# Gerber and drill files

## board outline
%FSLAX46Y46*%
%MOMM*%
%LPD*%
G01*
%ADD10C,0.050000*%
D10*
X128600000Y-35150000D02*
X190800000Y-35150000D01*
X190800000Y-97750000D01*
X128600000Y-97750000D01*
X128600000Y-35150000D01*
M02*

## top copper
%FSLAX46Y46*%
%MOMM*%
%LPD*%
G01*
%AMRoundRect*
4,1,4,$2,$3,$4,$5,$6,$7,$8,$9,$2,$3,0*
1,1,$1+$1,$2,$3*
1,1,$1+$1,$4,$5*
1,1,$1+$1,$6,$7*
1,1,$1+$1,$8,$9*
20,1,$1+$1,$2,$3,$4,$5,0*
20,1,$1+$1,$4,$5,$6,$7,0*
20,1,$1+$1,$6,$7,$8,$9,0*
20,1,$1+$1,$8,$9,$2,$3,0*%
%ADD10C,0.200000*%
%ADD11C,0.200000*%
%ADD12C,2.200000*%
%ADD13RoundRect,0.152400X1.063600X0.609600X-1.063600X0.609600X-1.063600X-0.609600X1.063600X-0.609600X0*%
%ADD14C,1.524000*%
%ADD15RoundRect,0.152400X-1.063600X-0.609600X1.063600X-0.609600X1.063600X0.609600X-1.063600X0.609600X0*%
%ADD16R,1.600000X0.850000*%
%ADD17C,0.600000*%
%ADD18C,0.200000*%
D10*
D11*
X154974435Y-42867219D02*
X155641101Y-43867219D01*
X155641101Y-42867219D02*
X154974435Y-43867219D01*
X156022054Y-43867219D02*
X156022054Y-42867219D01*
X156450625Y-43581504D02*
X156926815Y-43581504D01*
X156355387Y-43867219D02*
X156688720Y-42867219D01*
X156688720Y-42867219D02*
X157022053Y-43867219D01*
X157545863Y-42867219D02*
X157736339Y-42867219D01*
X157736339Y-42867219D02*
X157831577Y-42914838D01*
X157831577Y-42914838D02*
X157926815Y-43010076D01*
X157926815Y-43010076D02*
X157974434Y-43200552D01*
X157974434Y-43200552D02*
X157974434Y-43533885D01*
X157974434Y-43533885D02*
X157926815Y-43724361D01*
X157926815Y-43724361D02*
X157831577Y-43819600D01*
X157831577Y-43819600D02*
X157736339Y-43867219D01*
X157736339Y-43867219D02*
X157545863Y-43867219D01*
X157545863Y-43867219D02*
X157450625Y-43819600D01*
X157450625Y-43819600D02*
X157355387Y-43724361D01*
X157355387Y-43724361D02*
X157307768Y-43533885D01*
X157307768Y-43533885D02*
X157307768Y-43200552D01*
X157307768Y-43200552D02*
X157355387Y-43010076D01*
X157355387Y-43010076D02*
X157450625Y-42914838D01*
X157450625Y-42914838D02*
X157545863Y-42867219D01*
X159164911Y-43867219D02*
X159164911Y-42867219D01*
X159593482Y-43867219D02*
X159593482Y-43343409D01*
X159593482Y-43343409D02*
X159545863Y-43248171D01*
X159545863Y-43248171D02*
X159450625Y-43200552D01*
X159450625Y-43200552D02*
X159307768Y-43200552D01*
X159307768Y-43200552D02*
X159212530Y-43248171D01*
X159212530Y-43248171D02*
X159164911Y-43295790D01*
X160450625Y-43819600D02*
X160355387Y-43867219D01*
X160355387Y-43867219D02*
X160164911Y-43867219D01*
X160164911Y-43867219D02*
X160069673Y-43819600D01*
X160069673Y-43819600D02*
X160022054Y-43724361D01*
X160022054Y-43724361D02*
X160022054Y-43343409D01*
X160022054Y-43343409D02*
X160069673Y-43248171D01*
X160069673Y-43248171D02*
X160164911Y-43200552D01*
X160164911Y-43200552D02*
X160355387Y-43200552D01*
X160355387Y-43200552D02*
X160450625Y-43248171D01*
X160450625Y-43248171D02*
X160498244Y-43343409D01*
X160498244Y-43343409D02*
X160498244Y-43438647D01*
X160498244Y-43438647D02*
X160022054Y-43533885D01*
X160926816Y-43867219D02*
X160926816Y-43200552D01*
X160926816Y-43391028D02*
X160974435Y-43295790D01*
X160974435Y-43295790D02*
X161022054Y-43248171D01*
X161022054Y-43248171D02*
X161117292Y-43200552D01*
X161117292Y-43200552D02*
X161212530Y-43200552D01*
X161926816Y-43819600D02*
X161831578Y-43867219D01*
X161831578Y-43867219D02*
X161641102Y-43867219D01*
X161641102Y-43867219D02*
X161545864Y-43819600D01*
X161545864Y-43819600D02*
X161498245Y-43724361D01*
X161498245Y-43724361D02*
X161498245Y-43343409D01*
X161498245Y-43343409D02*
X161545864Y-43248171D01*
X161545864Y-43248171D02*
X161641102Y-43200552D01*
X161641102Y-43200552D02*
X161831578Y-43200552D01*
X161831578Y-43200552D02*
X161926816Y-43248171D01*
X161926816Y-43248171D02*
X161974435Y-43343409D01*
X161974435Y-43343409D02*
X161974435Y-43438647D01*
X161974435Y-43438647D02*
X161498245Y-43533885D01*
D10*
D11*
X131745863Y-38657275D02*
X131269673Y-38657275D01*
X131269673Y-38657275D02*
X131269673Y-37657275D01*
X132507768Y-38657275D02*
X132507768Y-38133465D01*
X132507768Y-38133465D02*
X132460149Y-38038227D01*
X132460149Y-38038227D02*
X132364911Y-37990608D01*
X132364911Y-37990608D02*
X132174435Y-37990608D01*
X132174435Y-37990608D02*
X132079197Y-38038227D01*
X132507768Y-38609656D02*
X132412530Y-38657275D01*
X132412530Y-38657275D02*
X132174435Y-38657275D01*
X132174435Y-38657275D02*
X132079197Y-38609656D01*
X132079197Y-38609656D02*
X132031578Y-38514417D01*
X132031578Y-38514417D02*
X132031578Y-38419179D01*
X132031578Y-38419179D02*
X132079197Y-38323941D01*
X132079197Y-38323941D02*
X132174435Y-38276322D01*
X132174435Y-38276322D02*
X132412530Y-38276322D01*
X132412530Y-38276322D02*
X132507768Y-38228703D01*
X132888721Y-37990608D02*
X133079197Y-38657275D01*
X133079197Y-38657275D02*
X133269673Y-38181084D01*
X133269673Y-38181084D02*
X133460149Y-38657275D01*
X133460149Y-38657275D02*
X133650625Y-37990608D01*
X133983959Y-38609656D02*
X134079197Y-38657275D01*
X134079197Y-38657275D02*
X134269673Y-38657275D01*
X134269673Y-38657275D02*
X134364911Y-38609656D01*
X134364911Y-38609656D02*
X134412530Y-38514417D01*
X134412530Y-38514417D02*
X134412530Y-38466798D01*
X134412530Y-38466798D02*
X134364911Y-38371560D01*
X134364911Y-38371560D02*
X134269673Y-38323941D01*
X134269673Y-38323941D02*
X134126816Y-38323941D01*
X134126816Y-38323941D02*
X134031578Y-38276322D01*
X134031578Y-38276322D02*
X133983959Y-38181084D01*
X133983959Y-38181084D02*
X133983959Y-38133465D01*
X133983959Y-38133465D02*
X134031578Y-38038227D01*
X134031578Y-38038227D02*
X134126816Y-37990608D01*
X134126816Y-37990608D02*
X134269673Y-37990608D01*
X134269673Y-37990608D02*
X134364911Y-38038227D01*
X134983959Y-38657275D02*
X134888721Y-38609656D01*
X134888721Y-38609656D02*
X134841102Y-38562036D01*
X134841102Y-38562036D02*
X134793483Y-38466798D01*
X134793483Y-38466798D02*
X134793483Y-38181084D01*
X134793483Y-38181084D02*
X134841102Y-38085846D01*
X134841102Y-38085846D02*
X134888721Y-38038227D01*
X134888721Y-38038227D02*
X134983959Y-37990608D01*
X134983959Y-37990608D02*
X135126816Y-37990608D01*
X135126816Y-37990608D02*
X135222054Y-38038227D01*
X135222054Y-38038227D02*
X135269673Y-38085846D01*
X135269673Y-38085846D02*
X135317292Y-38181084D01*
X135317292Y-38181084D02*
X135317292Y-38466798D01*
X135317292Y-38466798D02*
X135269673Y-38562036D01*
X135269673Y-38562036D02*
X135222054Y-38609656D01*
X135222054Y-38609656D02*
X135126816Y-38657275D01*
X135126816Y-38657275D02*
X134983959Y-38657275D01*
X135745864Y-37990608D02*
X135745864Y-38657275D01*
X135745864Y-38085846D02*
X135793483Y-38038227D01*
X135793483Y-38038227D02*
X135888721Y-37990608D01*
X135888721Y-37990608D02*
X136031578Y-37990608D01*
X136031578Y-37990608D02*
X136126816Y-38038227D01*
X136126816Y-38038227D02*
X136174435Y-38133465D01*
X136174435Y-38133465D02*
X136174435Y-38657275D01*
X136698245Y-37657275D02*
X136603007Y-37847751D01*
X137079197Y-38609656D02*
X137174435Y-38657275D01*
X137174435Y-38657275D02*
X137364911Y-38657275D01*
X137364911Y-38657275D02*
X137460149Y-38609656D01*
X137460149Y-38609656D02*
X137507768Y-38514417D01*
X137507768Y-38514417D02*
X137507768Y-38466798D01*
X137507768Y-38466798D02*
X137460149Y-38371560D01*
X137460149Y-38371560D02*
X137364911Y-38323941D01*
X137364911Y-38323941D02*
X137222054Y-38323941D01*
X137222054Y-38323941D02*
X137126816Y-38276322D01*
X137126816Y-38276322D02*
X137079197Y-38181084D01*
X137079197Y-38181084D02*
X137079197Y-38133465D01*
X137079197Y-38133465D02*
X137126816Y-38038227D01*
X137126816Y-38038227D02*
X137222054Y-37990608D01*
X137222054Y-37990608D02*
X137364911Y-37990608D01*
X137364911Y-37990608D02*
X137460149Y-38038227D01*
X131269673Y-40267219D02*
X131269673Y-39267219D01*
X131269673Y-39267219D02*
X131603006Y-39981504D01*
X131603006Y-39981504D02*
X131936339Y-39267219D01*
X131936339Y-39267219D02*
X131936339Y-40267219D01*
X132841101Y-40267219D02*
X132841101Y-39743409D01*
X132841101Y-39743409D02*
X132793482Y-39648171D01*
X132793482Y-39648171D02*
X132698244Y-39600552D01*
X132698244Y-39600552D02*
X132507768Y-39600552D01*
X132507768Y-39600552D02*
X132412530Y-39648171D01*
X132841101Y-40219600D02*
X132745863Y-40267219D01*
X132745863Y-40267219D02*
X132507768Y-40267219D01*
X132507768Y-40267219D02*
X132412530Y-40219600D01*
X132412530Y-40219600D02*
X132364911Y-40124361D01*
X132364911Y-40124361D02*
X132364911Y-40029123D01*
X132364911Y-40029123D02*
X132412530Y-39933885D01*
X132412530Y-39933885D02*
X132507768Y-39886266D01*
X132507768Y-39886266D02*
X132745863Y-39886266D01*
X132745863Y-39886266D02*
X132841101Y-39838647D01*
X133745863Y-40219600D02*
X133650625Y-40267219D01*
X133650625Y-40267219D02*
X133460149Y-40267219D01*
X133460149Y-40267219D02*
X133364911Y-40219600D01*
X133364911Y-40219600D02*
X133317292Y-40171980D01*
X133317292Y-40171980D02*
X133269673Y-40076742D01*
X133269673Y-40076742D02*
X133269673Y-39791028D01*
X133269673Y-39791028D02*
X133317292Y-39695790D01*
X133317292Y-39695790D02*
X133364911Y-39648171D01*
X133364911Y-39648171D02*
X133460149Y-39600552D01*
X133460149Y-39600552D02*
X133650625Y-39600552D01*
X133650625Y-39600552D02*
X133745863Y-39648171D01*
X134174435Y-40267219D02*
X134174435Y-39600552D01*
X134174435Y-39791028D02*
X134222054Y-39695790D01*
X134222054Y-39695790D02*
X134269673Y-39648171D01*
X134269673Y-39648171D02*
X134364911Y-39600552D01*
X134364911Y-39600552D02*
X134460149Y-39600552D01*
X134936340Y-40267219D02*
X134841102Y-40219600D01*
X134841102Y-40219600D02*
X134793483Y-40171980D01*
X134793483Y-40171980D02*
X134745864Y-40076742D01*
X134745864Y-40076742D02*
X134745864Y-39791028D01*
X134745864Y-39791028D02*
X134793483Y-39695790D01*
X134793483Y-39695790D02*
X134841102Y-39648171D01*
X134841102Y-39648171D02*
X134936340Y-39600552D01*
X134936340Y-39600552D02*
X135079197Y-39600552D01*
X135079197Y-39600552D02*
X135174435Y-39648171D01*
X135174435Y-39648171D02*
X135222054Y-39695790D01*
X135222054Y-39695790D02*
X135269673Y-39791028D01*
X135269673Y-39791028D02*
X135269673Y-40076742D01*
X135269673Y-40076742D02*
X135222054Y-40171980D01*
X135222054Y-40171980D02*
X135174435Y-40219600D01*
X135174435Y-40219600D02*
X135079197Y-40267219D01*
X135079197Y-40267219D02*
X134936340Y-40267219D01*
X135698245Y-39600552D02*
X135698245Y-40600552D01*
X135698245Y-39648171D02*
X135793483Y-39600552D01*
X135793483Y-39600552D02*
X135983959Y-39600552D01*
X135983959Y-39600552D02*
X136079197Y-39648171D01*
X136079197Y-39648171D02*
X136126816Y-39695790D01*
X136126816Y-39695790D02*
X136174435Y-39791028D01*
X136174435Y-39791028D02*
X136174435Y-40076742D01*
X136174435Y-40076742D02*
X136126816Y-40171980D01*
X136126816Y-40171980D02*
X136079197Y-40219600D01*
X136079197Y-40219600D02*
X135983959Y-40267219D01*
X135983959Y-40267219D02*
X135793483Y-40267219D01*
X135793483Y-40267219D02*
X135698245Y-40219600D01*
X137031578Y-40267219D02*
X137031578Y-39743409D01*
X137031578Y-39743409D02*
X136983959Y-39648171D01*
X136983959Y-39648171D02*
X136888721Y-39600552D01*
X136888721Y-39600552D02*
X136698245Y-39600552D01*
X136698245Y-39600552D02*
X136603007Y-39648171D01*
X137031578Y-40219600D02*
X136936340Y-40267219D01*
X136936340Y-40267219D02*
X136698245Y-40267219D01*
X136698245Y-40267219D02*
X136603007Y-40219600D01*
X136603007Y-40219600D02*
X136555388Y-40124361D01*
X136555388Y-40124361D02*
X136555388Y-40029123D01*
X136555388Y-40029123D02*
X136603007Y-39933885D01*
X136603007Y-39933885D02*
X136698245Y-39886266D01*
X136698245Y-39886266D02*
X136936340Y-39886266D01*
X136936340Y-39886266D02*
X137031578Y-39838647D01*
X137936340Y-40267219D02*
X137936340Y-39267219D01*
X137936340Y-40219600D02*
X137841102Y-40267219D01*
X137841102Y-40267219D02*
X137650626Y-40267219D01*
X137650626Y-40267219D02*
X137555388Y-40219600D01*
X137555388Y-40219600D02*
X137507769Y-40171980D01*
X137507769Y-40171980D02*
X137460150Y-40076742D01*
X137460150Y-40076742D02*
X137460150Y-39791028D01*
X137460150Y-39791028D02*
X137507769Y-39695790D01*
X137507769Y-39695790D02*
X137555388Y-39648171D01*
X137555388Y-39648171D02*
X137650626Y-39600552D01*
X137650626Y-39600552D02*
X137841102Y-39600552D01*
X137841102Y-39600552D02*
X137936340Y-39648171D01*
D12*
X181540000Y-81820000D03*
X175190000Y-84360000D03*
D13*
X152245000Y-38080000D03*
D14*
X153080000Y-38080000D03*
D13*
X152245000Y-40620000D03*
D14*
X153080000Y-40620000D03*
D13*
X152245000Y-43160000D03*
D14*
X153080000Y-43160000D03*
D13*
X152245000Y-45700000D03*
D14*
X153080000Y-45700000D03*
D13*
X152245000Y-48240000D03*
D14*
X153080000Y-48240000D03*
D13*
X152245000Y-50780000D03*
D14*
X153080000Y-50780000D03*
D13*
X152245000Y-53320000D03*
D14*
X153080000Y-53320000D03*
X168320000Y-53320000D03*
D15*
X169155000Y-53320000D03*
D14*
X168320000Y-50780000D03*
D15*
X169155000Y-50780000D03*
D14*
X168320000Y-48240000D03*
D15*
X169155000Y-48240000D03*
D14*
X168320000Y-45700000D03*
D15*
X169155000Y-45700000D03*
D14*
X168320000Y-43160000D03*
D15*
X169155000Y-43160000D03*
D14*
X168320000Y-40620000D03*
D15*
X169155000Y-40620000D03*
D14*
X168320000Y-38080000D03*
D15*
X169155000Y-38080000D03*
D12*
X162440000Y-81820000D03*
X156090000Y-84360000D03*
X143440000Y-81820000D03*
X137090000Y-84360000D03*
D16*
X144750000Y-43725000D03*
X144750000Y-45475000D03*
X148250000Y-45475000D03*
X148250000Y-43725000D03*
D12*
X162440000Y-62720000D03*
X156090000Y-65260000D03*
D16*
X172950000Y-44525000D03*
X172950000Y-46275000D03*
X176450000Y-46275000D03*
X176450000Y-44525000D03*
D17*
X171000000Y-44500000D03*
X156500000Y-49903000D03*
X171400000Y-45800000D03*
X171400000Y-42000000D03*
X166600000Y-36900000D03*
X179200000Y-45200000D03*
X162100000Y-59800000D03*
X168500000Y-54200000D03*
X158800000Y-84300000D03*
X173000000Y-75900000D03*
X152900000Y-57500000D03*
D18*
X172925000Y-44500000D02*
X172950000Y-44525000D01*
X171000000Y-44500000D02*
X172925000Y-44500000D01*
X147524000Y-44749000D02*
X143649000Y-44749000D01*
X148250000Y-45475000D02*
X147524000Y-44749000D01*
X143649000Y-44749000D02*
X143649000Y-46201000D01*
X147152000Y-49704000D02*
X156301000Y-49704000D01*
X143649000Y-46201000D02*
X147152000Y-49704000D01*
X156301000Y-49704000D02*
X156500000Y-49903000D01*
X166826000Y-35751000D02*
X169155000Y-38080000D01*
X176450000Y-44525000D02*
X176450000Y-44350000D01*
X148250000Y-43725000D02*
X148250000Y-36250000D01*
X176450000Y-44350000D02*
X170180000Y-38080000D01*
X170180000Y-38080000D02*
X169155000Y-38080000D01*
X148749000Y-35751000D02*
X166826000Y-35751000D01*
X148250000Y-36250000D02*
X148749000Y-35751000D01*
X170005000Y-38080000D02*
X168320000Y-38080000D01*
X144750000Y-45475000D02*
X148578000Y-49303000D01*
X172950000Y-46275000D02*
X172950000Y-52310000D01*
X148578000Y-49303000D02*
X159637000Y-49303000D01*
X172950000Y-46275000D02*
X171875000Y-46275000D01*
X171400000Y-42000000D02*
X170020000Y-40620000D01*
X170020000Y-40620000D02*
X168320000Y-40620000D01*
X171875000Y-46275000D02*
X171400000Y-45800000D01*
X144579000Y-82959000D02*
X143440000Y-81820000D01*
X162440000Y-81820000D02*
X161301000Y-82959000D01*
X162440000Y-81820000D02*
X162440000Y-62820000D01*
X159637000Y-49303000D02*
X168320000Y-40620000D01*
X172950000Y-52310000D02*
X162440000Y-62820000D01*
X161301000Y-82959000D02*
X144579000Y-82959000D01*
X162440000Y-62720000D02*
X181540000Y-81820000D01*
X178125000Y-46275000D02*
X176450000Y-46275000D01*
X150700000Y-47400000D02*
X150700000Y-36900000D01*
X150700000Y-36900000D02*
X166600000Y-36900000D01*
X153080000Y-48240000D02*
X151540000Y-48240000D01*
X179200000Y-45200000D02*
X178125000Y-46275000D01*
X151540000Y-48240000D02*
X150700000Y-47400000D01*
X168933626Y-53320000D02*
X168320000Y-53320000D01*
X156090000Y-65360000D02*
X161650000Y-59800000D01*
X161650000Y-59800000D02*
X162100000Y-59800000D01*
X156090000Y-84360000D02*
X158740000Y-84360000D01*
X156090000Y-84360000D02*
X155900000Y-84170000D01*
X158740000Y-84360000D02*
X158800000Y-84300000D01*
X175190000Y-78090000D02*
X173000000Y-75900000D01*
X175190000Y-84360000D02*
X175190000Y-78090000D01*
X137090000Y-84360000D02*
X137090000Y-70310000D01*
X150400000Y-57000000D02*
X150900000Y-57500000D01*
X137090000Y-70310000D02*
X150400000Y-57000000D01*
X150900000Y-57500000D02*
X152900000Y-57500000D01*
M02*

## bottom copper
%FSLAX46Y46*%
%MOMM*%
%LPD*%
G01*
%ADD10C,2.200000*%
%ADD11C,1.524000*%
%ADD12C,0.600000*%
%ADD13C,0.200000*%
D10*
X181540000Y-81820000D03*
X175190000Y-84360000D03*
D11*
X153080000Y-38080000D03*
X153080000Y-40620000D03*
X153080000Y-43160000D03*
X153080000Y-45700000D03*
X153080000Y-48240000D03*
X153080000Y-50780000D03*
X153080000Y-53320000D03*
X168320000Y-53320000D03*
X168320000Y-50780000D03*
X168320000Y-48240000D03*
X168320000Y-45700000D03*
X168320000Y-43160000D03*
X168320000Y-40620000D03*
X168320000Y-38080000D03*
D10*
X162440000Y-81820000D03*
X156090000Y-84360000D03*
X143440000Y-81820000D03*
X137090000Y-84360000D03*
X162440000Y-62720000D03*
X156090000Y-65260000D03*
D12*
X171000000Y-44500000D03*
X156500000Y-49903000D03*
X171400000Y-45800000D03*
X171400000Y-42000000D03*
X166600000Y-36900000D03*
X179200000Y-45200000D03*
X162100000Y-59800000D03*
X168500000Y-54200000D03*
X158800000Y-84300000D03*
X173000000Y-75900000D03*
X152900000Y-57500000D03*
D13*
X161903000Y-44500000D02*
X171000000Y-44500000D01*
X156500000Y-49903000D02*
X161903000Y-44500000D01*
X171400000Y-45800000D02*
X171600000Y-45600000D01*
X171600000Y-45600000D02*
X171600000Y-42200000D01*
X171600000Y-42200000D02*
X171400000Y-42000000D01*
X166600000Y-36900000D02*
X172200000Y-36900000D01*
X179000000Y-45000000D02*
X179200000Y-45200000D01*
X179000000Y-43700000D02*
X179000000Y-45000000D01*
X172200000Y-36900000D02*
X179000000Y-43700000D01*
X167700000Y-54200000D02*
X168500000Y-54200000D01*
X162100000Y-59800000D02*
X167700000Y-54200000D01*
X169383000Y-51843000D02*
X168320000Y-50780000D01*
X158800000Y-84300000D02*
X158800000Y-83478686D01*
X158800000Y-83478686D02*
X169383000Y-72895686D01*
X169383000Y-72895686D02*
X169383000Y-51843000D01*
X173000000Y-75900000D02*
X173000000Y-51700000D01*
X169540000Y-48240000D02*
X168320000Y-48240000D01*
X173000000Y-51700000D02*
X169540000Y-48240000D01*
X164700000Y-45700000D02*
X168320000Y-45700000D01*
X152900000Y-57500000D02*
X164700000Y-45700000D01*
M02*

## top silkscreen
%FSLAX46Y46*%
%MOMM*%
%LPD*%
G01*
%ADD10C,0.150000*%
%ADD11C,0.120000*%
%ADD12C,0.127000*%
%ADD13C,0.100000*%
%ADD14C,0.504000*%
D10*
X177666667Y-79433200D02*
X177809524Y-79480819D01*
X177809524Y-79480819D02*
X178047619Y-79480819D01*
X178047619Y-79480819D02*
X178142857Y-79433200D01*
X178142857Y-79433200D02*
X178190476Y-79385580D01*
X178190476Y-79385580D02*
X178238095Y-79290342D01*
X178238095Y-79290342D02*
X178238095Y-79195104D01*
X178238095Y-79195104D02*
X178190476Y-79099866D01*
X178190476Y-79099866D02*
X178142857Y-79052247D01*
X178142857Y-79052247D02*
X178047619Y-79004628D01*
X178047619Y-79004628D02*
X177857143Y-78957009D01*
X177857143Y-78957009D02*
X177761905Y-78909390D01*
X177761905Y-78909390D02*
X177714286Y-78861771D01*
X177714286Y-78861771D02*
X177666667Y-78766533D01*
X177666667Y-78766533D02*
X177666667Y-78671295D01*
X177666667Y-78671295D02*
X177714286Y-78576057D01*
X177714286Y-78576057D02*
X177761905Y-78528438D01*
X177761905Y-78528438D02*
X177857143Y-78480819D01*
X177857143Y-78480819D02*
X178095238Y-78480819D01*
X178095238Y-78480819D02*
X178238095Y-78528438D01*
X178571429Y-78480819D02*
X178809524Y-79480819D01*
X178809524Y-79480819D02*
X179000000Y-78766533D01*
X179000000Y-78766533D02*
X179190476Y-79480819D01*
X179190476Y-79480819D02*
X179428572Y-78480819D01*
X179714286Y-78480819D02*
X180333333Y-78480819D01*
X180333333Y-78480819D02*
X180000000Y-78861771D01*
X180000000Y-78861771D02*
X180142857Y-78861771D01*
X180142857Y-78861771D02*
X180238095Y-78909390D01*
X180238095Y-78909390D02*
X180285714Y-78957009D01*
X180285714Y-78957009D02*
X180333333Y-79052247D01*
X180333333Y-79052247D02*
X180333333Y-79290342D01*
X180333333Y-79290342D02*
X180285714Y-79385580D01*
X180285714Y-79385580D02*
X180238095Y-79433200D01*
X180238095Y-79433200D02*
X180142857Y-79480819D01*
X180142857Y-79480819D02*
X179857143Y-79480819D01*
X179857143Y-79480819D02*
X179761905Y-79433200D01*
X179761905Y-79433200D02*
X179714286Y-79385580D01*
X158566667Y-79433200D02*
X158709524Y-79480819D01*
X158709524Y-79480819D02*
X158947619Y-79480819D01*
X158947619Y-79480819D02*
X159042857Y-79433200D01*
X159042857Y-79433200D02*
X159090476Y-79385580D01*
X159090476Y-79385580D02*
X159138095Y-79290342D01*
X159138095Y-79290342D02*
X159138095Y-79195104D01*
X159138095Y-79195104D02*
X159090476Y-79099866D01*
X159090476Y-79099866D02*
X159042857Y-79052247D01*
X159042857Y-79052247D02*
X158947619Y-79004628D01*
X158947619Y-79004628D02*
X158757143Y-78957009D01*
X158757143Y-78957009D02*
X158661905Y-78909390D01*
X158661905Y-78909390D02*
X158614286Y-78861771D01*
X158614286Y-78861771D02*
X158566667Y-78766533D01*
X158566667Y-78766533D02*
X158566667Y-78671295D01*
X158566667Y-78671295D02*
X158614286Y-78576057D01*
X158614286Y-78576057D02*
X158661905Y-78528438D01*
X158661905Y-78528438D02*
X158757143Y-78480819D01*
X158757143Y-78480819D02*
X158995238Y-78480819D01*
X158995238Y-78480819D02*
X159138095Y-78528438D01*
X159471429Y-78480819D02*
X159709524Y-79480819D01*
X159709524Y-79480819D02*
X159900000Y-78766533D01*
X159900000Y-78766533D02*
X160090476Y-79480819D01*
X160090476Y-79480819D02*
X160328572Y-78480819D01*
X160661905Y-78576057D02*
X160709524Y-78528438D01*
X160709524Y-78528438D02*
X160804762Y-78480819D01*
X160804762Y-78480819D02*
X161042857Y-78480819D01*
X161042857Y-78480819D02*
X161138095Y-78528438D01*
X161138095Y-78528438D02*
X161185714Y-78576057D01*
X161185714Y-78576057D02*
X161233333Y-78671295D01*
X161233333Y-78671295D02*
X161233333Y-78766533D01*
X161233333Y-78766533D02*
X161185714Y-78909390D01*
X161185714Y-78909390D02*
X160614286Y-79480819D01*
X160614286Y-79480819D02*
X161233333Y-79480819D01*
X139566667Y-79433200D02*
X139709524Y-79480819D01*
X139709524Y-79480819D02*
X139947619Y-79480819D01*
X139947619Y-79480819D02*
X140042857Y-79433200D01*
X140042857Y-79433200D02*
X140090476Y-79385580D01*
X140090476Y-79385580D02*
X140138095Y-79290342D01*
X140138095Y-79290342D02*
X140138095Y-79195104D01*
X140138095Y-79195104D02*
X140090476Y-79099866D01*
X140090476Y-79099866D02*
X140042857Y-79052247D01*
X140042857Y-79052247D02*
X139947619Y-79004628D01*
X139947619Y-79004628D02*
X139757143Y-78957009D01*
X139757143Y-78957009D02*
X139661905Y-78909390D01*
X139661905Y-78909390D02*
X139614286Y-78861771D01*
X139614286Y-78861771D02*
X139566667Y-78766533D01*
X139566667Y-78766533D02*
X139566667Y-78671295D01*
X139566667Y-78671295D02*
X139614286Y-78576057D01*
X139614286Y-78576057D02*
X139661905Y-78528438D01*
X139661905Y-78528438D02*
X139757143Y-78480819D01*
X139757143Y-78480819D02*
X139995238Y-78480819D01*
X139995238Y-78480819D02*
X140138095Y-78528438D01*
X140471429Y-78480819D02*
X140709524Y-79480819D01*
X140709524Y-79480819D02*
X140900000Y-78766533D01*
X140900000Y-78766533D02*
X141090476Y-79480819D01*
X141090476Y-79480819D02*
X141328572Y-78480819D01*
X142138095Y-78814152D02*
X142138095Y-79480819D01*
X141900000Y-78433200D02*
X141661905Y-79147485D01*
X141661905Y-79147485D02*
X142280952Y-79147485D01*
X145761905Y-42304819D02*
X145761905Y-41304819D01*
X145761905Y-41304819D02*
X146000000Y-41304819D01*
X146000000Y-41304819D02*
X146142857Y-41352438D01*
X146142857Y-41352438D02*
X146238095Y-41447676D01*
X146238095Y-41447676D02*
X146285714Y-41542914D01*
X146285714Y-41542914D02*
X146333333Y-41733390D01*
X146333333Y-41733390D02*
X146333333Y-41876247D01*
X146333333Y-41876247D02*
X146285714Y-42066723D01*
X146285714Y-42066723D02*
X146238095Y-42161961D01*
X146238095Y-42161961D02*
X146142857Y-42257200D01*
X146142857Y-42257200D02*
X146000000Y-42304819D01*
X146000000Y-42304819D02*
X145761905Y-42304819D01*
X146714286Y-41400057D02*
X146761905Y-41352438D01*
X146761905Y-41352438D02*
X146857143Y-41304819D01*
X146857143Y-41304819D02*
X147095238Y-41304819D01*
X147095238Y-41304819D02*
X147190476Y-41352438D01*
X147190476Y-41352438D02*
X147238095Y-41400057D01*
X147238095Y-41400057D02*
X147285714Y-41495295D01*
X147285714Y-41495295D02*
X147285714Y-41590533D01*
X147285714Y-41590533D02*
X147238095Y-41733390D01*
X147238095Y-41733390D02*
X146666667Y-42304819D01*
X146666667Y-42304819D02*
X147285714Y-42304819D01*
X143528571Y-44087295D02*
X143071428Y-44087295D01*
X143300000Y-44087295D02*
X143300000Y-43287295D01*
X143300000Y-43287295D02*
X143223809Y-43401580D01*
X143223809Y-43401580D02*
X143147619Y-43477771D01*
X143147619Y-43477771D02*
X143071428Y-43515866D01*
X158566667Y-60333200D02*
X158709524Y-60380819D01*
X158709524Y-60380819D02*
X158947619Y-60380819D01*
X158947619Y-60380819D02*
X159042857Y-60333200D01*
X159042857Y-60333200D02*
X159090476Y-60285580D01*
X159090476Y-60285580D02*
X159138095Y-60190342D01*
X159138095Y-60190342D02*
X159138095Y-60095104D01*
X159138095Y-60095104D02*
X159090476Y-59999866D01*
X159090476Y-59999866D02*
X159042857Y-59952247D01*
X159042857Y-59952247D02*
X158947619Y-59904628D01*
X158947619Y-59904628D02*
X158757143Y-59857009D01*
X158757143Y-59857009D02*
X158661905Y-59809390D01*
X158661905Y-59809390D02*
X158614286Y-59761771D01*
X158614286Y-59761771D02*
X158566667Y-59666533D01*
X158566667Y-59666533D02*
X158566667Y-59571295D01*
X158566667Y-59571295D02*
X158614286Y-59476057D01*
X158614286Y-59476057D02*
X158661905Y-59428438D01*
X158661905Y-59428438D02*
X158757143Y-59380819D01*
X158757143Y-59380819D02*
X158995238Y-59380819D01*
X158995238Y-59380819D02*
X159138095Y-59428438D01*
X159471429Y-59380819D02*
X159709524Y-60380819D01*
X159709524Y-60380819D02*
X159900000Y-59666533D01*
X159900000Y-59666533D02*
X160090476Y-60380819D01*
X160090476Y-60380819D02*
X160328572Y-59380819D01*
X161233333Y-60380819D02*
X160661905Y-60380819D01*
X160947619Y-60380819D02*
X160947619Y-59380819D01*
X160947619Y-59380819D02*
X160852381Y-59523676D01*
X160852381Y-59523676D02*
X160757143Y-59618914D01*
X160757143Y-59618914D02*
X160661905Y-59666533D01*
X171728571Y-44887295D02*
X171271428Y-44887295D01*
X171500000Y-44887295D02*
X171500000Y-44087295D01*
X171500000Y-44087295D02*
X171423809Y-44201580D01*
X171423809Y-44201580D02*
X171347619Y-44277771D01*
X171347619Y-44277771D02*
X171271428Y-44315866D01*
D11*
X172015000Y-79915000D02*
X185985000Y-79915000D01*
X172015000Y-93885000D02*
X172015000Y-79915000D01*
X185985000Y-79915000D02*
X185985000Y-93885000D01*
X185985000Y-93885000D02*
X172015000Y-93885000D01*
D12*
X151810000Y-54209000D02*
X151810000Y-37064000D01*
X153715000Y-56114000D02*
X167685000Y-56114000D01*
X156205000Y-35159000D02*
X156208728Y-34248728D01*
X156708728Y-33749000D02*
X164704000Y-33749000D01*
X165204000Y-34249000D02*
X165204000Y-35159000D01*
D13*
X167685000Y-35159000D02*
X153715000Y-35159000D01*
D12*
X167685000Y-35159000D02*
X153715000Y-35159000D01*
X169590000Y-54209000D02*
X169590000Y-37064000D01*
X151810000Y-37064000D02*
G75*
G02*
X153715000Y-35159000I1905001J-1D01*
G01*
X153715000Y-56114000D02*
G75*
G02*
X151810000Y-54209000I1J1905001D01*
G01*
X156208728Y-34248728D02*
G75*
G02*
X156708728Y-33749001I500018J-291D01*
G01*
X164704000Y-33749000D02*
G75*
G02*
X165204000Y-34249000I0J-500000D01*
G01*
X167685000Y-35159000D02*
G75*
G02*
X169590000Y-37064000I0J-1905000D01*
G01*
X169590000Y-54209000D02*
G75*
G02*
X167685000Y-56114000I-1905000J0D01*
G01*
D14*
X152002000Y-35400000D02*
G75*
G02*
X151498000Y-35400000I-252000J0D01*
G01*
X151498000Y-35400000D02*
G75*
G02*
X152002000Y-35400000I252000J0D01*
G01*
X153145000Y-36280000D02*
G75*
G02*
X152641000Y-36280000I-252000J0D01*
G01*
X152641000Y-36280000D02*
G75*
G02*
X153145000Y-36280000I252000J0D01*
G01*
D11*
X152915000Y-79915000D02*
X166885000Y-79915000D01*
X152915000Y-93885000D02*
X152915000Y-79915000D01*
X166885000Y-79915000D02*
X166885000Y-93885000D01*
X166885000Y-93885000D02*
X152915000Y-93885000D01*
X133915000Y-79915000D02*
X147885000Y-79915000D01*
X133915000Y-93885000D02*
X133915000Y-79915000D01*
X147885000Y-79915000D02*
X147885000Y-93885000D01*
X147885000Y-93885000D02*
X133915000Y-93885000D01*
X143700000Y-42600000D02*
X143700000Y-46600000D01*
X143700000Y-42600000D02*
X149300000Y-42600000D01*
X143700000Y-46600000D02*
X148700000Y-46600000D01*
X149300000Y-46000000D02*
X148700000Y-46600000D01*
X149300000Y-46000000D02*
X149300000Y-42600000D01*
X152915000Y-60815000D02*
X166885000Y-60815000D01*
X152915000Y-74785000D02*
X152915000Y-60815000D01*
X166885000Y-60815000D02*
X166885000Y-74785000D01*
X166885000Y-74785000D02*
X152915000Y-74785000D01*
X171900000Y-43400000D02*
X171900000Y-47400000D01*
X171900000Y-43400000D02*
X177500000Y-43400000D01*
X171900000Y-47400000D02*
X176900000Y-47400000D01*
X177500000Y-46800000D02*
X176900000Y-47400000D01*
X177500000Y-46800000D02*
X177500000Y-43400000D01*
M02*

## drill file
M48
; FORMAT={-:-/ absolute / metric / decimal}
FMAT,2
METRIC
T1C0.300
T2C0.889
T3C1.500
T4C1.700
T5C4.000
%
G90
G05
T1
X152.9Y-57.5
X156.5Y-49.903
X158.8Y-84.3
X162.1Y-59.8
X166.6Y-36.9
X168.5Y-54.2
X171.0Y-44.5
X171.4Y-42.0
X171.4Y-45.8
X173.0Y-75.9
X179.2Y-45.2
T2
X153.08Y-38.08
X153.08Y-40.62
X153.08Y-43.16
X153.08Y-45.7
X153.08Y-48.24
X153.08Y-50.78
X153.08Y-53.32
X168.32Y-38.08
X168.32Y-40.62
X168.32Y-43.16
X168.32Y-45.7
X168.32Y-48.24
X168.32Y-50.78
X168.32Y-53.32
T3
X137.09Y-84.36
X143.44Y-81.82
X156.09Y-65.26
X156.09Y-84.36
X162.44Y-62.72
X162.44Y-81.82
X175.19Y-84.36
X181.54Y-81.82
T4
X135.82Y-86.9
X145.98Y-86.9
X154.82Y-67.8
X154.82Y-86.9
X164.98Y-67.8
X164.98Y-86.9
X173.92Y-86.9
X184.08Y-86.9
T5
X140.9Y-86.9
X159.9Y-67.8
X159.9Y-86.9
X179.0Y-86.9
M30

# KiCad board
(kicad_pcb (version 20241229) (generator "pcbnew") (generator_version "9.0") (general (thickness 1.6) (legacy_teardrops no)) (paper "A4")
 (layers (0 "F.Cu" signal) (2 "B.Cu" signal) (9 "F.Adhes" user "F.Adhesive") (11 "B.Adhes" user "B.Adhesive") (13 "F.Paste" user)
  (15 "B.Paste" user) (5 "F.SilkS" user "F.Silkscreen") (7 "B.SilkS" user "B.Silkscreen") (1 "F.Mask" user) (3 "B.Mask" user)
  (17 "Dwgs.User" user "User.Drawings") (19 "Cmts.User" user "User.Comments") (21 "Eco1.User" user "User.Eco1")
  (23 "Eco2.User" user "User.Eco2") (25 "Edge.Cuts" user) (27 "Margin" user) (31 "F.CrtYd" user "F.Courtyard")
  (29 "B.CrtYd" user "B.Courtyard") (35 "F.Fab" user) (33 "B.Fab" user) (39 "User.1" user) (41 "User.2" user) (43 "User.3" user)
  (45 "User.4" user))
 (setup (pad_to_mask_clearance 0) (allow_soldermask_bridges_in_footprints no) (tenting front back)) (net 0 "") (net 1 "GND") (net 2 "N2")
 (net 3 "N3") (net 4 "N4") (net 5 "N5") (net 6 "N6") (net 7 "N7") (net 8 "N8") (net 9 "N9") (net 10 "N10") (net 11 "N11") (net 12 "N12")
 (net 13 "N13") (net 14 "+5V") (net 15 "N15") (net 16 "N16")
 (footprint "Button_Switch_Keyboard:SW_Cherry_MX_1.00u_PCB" (layer "F.Cu") (at 181.54 81.82)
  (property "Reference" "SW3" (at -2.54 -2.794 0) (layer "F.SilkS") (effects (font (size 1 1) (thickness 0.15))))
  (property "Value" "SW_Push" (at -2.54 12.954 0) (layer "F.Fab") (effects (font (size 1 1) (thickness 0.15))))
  (fp_line (start -9.525 -1.905) (end 4.445 -1.905) (stroke (width 0.12) (type solid)) (layer "F.SilkS"))
  (fp_line (start -9.525 12.065) (end -9.525 -1.905) (stroke (width 0.12) (type solid)) (layer "F.SilkS"))
  (fp_line (start 4.445 -1.905) (end 4.445 12.065) (stroke (width 0.12) (type solid)) (layer "F.SilkS"))
  (fp_line (start 4.445 12.065) (end -9.525 12.065) (stroke (width 0.12) (type solid)) (layer "F.SilkS"))
  (pad "" np_thru_hole circle (at -7.62 5.08) (size 1.7 1.7) (drill 1.7) (layers "*.Cu" "*.Mask"))
  (pad "" np_thru_hole circle (at -2.54 5.08) (size 4 4) (drill 4) (layers "*.Cu" "*.Mask"))
  (pad "" np_thru_hole circle (at 2.54 5.08) (size 1.7 1.7) (drill 1.7) (layers "*.Cu" "*.Mask"))
  (pad "1" thru_hole circle (at 0 0) (size 2.2 2.2) (drill 1.5) (layers "*.Cu" "*.Mask") (remove_unused_layers no) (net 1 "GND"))
  (pad "2" thru_hole circle (at -6.35 2.54) (size 2.2 2.2) (drill 1.5) (layers "*.Cu" "*.Mask") (remove_unused_layers no) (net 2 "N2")))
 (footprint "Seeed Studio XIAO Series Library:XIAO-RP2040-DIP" (layer "F.Cu") (at 160.7 45.7)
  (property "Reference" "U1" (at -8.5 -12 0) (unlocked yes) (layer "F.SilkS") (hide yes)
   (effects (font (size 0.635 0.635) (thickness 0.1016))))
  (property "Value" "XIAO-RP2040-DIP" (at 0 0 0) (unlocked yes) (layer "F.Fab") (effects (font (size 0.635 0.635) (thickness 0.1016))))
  (fp_line (start -8.89 8.509) (end -8.89 -8.636) (stroke (width 0.127) (type solid)) (layer "F.SilkS"))
  (fp_line (start -6.985 10.414) (end 6.985 10.414) (stroke (width 0.127) (type solid)) (layer "F.SilkS"))
  (fp_line (start -4.495 -10.541) (end -4.491272 -11.451272) (stroke (width 0.127) (type solid)) (layer "F.SilkS"))
  (fp_line (start -3.991272 -11.951) (end 4.004 -11.951) (stroke (width 0.127) (type solid)) (layer "F.SilkS"))
  (fp_line (start 4.504 -11.451) (end 4.504 -10.541) (stroke (width 0.127) (type solid)) (layer "F.SilkS"))
  (fp_line (start 6.985 -10.541) (end -6.985 -10.541) (stroke (width 0.1) (type solid)) (layer "F.SilkS"))
  (fp_line (start 6.985 -10.541) (end -6.985 -10.541) (stroke (width 0.127) (type solid)) (layer "F.SilkS"))
  (fp_line (start 8.89 8.509) (end 8.89 -8.636) (stroke (width 0.127) (type solid)) (layer "F.SilkS"))
  (fp_arc (start -8.89 -8.636) (mid -8.332038 -9.983038) (end -6.985 -10.541) (stroke (width 0.127) (type solid)) (layer "F.SilkS"))
  (fp_arc (start -6.985 10.414) (mid -8.332038 9.856038) (end -8.89 8.509) (stroke (width 0.127) (type solid)) (layer "F.SilkS"))
  (fp_arc (start -4.491272 -11.451272) (mid -4.344728 -11.80464) (end -3.991272 -11.951) (stroke (width 0.127) (type default))
   (layer "F.SilkS"))
  (fp_arc (start 4.004 -11.951) (mid 4.357553 -11.804553) (end 4.504 -11.451) (stroke (width 0.127) (type default)) (layer "F.SilkS"))
  (fp_arc (start 6.985 -10.541) (mid 8.332038 -9.983038) (end 8.89 -8.636) (stroke (width 0.127) (type solid)) (layer "F.SilkS"))
  (fp_arc (start 8.89 8.509) (mid 8.332038 9.856038) (end 6.985 10.414) (stroke (width 0.127) (type solid)) (layer "F.SilkS"))
  (fp_circle (center -8.95 -10.3) (end -8.95 -10.554) (stroke (width 0.5) (type solid)) (fill yes) (layer "F.SilkS"))
  (fp_circle (center -7.807 -9.42) (end -7.807 -9.674) (stroke (width 0.5) (type solid)) (fill yes) (layer "F.SilkS"))
  (pad "1" smd roundrect (at -8.455 -7.62 180) (size 2.432 1.524) (layers "F.Cu" "F.Mask") (roundrect_rratio 0.1) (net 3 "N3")
   (thermal_bridge_angle 45))
  (pad "1" thru_hole circle (at -7.62 -7.62 180) (size 1.524 1.524) (drill 0.889) (layers "*.Cu" "*.Mask") (remove_unused_layers no)
   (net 3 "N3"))
  (pad "2" smd roundrect (at -8.455 -5.08 180) (size 2.432 1.524) (layers "F.Cu" "F.Mask") (roundrect_rratio 0.1) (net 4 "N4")
   (thermal_bridge_angle 45))
  (pad "2" thru_hole circle (at -7.62 -5.08 180) (size 1.524 1.524) (drill 0.889) (layers "*.Cu" "*.Mask") (remove_unused_layers no)
   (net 4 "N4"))
  (pad "3" smd roundrect (at -8.455 -2.54 180) (size 2.432 1.524) (layers "F.Cu" "F.Mask") (roundrect_rratio 0.1) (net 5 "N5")
   (thermal_bridge_angle 45))
  (pad "3" thru_hole circle (at -7.62 -2.54 180) (size 1.524 1.524) (drill 0.889) (layers "*.Cu" "*.Mask") (remove_unused_layers no)
   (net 5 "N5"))
  (pad "4" smd roundrect (at -8.455 0 180) (size 2.432 1.524) (layers "F.Cu" "F.Mask") (roundrect_rratio 0.1) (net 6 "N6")
   (thermal_bridge_angle 45))
  (pad "4" thru_hole circle (at -7.62 0 180) (size 1.524 1.524) (drill 0.889) (layers "*.Cu" "*.Mask") (remove_unused_layers no)
   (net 6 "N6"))
  (pad "5" smd roundrect (at -8.455 2.54 180) (size 2.432 1.524) (layers "F.Cu" "F.Mask") (roundrect_rratio 0.1) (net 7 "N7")
   (thermal_bridge_angle 45))
  (pad "5" thru_hole circle (at -7.62 2.54 180) (size 1.524 1.524) (drill 0.889) (layers "*.Cu" "*.Mask") (remove_unused_layers no)
   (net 7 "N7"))
  (pad "6" smd roundrect (at -8.455 5.08 180) (size 2.432 1.524) (layers "F.Cu" "F.Mask") (roundrect_rratio 0.1) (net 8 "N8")
   (thermal_bridge_angle 45))
  (pad "6" thru_hole circle (at -7.62 5.08 180) (size 1.524 1.524) (drill 0.889) (layers "*.Cu" "*.Mask") (remove_unused_layers no)
   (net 8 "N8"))
  (pad "7" smd roundrect (at -8.455 7.62 180) (size 2.432 1.524) (layers "F.Cu" "F.Mask") (roundrect_rratio 0.1) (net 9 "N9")
   (thermal_bridge_angle 45))
  (pad "7" thru_hole circle (at -7.62 7.62 180) (size 1.524 1.524) (drill 0.889) (layers "*.Cu" "*.Mask") (remove_unused_layers no)
   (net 9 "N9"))
  (pad "8" thru_hole circle (at 7.62 7.62) (size 1.524 1.524) (drill 0.889) (layers "*.Cu" "*.Mask") (remove_unused_layers no)
   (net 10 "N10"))
  (pad "8" smd roundrect (at 8.455 7.62) (size 2.432 1.524) (layers "F.Cu" "F.Mask") (roundrect_rratio 0.1) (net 10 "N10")
   (thermal_bridge_angle 45))
  (pad "9" thru_hole circle (at 7.62 5.08) (size 1.524 1.524) (drill 0.889) (layers "*.Cu" "*.Mask") (remove_unused_layers no)
   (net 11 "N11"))
  (pad "9" smd roundrect (at 8.455 5.08) (size 2.432 1.524) (layers "F.Cu" "F.Mask") (roundrect_rratio 0.1) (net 11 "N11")
   (thermal_bridge_angle 45))
  (pad "10" thru_hole circle (at 7.62 2.54) (size 1.524 1.524) (drill 0.889) (layers "*.Cu" "*.Mask") (remove_unused_layers no) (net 2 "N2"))
  (pad "10" smd roundrect (at 8.455 2.54) (size 2.432 1.524) (layers "F.Cu" "F.Mask") (roundrect_rratio 0.1) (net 2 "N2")
   (thermal_bridge_angle 45))
  (pad "11" thru_hole circle (at 7.62 0) (size 1.524 1.524) (drill 0.889) (layers "*.Cu" "*.Mask") (remove_unused_layers no) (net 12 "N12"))
  (pad "11" smd roundrect (at 8.455 0) (size 2.432 1.524) (layers "F.Cu" "F.Mask") (roundrect_rratio 0.1) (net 12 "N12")
   (thermal_bridge_angle 45))
  (pad "12" thru_hole circle (at 7.62 -2.54) (size 1.524 1.524) (drill 0.889) (layers "*.Cu" "*.Mask") (remove_unused_layers no)
   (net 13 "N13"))
  (pad "12" smd roundrect (at 8.455 -2.54) (size 2.432 1.524) (layers "F.Cu" "F.Mask") (roundrect_rratio 0.1) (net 13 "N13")
   (thermal_bridge_angle 45))
  (pad "13" thru_hole circle (at 7.62 -5.08) (size 1.524 1.524) (drill 0.889) (layers "*.Cu" "*.Mask") (remove_unused_layers no)
   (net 1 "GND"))
  (pad "13" smd roundrect (at 8.455 -5.08) (size 2.432 1.524) (layers "F.Cu" "F.Mask") (roundrect_rratio 0.1) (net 1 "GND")
   (thermal_bridge_angle 45))
  (pad "14" thru_hole circle (at 7.62 -7.62) (size 1.524 1.524) (drill 0.889) (layers "*.Cu" "*.Mask") (remove_unused_layers no)
   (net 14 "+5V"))
  (pad "14" smd roundrect (at 8.455 -7.62) (size 2.432 1.524) (layers "F.Cu" "F.Mask") (roundrect_rratio 0.1) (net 14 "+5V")
   (thermal_bridge_angle 45)))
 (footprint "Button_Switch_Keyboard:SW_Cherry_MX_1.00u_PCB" (layer "F.Cu") (at 162.44 81.82)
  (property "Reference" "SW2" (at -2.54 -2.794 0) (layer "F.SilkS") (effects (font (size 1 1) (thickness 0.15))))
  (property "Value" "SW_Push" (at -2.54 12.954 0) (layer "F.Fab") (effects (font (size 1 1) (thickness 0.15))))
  (fp_line (start -9.525 -1.905) (end 4.445 -1.905) (stroke (width 0.12) (type solid)) (layer "F.SilkS"))
  (fp_line (start -9.525 12.065) (end -9.525 -1.905) (stroke (width 0.12) (type solid)) (layer "F.SilkS"))
  (fp_line (start 4.445 -1.905) (end 4.445 12.065) (stroke (width 0.12) (type solid)) (layer "F.SilkS"))
  (fp_line (start 4.445 12.065) (end -9.525 12.065) (stroke (width 0.12) (type solid)) (layer "F.SilkS"))
  (pad "" np_thru_hole circle (at -7.62 5.08) (size 1.7 1.7) (drill 1.7) (layers "*.Cu" "*.Mask"))
  (pad "" np_thru_hole circle (at -2.54 5.08) (size 4 4) (drill 4) (layers "*.Cu" "*.Mask"))
  (pad "" np_thru_hole circle (at 2.54 5.08) (size 1.7 1.7) (drill 1.7) (layers "*.Cu" "*.Mask"))
  (pad "1" thru_hole circle (at 0 0) (size 2.2 2.2) (drill 1.5) (layers "*.Cu" "*.Mask") (remove_unused_layers no) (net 1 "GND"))
  (pad "2" thru_hole circle (at -6.35 2.54) (size 2.2 2.2) (drill 1.5) (layers "*.Cu" "*.Mask") (remove_unused_layers no) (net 11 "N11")))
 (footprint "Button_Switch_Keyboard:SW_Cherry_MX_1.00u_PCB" (layer "F.Cu") (at 143.44 81.82)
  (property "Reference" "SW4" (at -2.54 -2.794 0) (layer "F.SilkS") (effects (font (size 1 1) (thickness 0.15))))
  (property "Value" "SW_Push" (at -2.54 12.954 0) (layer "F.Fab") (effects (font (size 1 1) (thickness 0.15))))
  (fp_line (start -9.525 -1.905) (end 4.445 -1.905) (stroke (width 0.12) (type solid)) (layer "F.SilkS"))
  (fp_line (start -9.525 12.065) (end -9.525 -1.905) (stroke (width 0.12) (type solid)) (layer "F.SilkS"))
  (fp_line (start 4.445 -1.905) (end 4.445 12.065) (stroke (width 0.12) (type solid)) (layer "F.SilkS"))
  (fp_line (start 4.445 12.065) (end -9.525 12.065) (stroke (width 0.12) (type solid)) (layer "F.SilkS"))
  (pad "" np_thru_hole circle (at -7.62 5.08) (size 1.7 1.7) (drill 1.7) (layers "*.Cu" "*.Mask"))
  (pad "" np_thru_hole circle (at -2.54 5.08) (size 4 4) (drill 4) (layers "*.Cu" "*.Mask"))
  (pad "" np_thru_hole circle (at 2.54 5.08) (size 1.7 1.7) (drill 1.7) (layers "*.Cu" "*.Mask"))
  (pad "1" thru_hole circle (at 0 0) (size 2.2 2.2) (drill 1.5) (layers "*.Cu" "*.Mask") (remove_unused_layers no) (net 1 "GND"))
  (pad "2" thru_hole circle (at -6.35 2.54) (size 2.2 2.2) (drill 1.5) (layers "*.Cu" "*.Mask") (remove_unused_layers no) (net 12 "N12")))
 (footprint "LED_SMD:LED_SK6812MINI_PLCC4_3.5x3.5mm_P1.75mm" (layer "F.Cu") (at 146.5 44.6)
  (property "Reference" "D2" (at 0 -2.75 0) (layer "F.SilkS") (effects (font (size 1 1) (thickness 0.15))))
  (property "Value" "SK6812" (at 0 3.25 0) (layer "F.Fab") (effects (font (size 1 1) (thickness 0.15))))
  (fp_line (start -2.8 -2) (end -2.8 2) (stroke (width 0.12) (type default)) (layer "F.SilkS"))
  (fp_line (start -2.8 -2) (end 2.8 -2) (stroke (width 0.12) (type solid)) (layer "F.SilkS"))
  (fp_line (start -2.8 2) (end 2.2 2) (stroke (width 0.12) (type solid)) (layer "F.SilkS"))
  (fp_line (start 2.8 1.4) (end 2.2 2) (stroke (width 0.12) (type default)) (layer "F.SilkS"))
  (fp_line (start 2.8 1.4) (end 2.8 -2) (stroke (width 0.12) (type solid)) (layer "F.SilkS"))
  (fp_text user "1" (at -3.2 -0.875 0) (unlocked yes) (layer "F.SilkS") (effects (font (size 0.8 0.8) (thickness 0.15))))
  (pad "1" smd rect (at -1.75 -0.875) (size 1.6 0.85) (layers "F.Cu" "F.Mask" "F.Paste") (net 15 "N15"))
  (pad "2" smd rect (at -1.75 0.875) (size 1.6 0.85) (layers "F.Cu" "F.Mask" "F.Paste") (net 1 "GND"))
  (pad "3" smd rect (at 1.75 0.875) (size 1.6 0.85) (layers "F.Cu" "F.Mask" "F.Paste") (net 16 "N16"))
  (pad "4" smd rect (at 1.75 -0.875) (size 1.6 0.85) (layers "F.Cu" "F.Mask" "F.Paste") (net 14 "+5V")))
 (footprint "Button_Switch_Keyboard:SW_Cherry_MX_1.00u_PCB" (layer "F.Cu") (at 162.44 62.72)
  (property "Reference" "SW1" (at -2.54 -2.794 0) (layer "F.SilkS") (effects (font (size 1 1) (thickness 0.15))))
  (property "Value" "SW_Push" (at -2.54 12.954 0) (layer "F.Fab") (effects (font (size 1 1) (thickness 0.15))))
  (fp_line (start -9.525 -1.905) (end 4.445 -1.905) (stroke (width 0.12) (type solid)) (layer "F.SilkS"))
  (fp_line (start -9.525 12.065) (end -9.525 -1.905) (stroke (width 0.12) (type solid)) (layer "F.SilkS"))
  (fp_line (start 4.445 -1.905) (end 4.445 12.065) (stroke (width 0.12) (type solid)) (layer "F.SilkS"))
  (fp_line (start 4.445 12.065) (end -9.525 12.065) (stroke (width 0.12) (type solid)) (layer "F.SilkS"))
  (pad "" np_thru_hole circle (at -7.62 5.08) (size 1.7 1.7) (drill 1.7) (layers "*.Cu" "*.Mask"))
  (pad "" np_thru_hole circle (at -2.54 5.08) (size 4 4) (drill 4) (layers "*.Cu" "*.Mask"))
  (pad "" np_thru_hole circle (at 2.54 5.08) (size 1.7 1.7) (drill 1.7) (layers "*.Cu" "*.Mask"))
  (pad "1" thru_hole circle (at 0 0) (size 2.2 2.2) (drill 1.5) (layers "*.Cu" "*.Mask") (remove_unused_layers no) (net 1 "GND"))
  (pad "2" thru_hole circle (at -6.35 2.54) (size 2.2 2.2) (drill 1.5) (layers "*.Cu" "*.Mask") (remove_unused_layers no) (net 10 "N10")))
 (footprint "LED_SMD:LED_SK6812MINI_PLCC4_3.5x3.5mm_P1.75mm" (layer "F.Cu") (at 174.7 45.4)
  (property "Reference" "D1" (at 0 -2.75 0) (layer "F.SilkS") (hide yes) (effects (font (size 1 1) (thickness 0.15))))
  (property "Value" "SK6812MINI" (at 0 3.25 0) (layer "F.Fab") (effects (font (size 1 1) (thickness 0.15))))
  (fp_line (start -2.8 -2) (end -2.8 2) (stroke (width 0.12) (type default)) (layer "F.SilkS"))
  (fp_line (start -2.8 -2) (end 2.8 -2) (stroke (width 0.12) (type solid)) (layer "F.SilkS"))
  (fp_line (start -2.8 2) (end 2.2 2) (stroke (width 0.12) (type solid)) (layer "F.SilkS"))
  (fp_line (start 2.8 1.4) (end 2.2 2) (stroke (width 0.12) (type default)) (layer "F.SilkS"))
  (fp_line (start 2.8 1.4) (end 2.8 -2) (stroke (width 0.12) (type solid)) (layer "F.SilkS"))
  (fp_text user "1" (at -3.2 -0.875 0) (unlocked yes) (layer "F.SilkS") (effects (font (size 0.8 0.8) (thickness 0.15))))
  (pad "1" smd rect (at -1.75 -0.875) (size 1.6 0.85) (layers "F.Cu" "F.Mask" "F.Paste") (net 16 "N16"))
  (pad "2" smd rect (at -1.75 0.875) (size 1.6 0.85) (layers "F.Cu" "F.Mask" "F.Paste") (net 1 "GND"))
  (pad "3" smd rect (at 1.75 0.875) (size 1.6 0.85) (layers "F.Cu" "F.Mask" "F.Paste") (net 7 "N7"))
  (pad "4" smd rect (at 1.75 -0.875) (size 1.6 0.85) (layers "F.Cu" "F.Mask" "F.Paste") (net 14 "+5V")))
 (gr_rect (start 128.6 35.15) (end 190.8 97.75) (stroke (width 0.05) (type default)) (fill no) (layer "Edge.Cuts"))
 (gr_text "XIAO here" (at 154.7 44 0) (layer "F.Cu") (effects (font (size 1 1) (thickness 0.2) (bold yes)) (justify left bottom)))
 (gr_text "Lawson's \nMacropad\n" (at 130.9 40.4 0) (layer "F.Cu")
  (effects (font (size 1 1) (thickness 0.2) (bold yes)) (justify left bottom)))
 (segment (start 172.925 44.5) (end 172.95 44.525) (width 0.2) (layer "F.Cu") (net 16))
 (segment (start 171 44.5) (end 172.925 44.5) (width 0.2) (layer "F.Cu") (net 16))
 (segment (start 147.524 44.749) (end 143.649 44.749) (width 0.2) (layer "F.Cu") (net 16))
 (segment (start 148.25 45.475) (end 147.524 44.749) (width 0.2) (layer "F.Cu") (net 16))
 (segment (start 143.649 44.749) (end 143.649 46.201) (width 0.2) (layer "F.Cu") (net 16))
 (segment (start 147.152 49.704) (end 156.301 49.704) (width 0.2) (layer "F.Cu") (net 16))
 (segment (start 143.649 46.201) (end 147.152 49.704) (width 0.2) (layer "F.Cu") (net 16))
 (segment (start 156.301 49.704) (end 156.5 49.903) (width 0.2) (layer "F.Cu") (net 16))
 (via (at 171 44.5) (size 0.6) (drill 0.3) (layers "F.Cu" "B.Cu") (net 16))
 (via (at 156.5 49.903) (size 0.6) (drill 0.3) (layers "F.Cu" "B.Cu") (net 16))
 (segment (start 161.903 44.5) (end 171 44.5) (width 0.2) (layer "B.Cu") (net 16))
 (segment (start 156.5 49.903) (end 161.903 44.5) (width 0.2) (layer "B.Cu") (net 16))
 (segment (start 166.826 35.751) (end 169.155 38.08) (width 0.2) (layer "F.Cu") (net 14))
 (segment (start 176.45 44.525) (end 176.45 44.35) (width 0.2) (layer "F.Cu") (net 14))
 (segment (start 148.25 43.725) (end 148.25 36.25) (width 0.2) (layer "F.Cu") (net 14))
 (segment (start 176.45 44.35) (end 170.18 38.08) (width 0.2) (layer "F.Cu") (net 14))
 (segment (start 170.18 38.08) (end 169.155 38.08) (width 0.2) (layer "F.Cu") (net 14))
 (segment (start 148.749 35.751) (end 166.826 35.751) (width 0.2) (layer "F.Cu") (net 14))
 (segment (start 148.25 36.25) (end 148.749 35.751) (width 0.2) (layer "F.Cu") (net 14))
 (segment (start 170.005 38.08) (end 168.32 38.08) (width 0.2) (layer "F.Cu") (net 14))
 (segment (start 144.75 45.475) (end 148.578 49.303) (width 0.2) (layer "F.Cu") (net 1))
 (segment (start 172.95 46.275) (end 172.95 52.31) (width 0.2) (layer "F.Cu") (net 1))
 (segment (start 148.578 49.303) (end 159.637 49.303) (width 0.2) (layer "F.Cu") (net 1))
 (segment (start 172.95 46.275) (end 171.875 46.275) (width 0.2) (layer "F.Cu") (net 1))
 (segment (start 171.4 42) (end 170.02 40.62) (width 0.2) (layer "F.Cu") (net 1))
 (segment (start 170.02 40.62) (end 168.32 40.62) (width 0.2) (layer "F.Cu") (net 1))
 (segment (start 171.875 46.275) (end 171.4 45.8) (width 0.2) (layer "F.Cu") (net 1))
 (segment (start 144.579 82.959) (end 143.44 81.82) (width 0.2) (layer "F.Cu") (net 1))
 (segment (start 162.44 81.82) (end 161.301 82.959) (width 0.2) (layer "F.Cu") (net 1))
 (segment (start 162.44 81.82) (end 162.44 62.82) (width 0.2) (layer "F.Cu") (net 1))
 (segment (start 159.637 49.303) (end 168.32 40.62) (width 0.2) (layer "F.Cu") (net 1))
 (segment (start 172.95 52.31) (end 162.44 62.82) (width 0.2) (layer "F.Cu") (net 1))
 (segment (start 161.301 82.959) (end 144.579 82.959) (width 0.2) (layer "F.Cu") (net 1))
 (segment (start 162.44 62.72) (end 181.54 81.82) (width 0.2) (layer "F.Cu") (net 1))
 (via (at 171.4 45.8) (size 0.6) (drill 0.3) (layers "F.Cu" "B.Cu") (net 1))
 (via (at 171.4 42) (size 0.6) (drill 0.3) (layers "F.Cu" "B.Cu") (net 1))
 (segment (start 171.4 45.8) (end 171.6 45.6) (width 0.2) (layer "B.Cu") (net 1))
 (segment (start 171.6 45.6) (end 171.6 42.2) (width 0.2) (layer "B.Cu") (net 1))
 (segment (start 171.6 42.2) (end 171.4 42) (width 0.2) (layer "B.Cu") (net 1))
 (segment (start 178.125 46.275) (end 176.45 46.275) (width 0.2) (layer "F.Cu") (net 7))
 (segment (start 150.7 47.4) (end 150.7 36.9) (width 0.2) (layer "F.Cu") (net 7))
 (segment (start 150.7 36.9) (end 166.6 36.9) (width 0.2) (layer "F.Cu") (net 7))
 (segment (start 153.08 48.24) (end 151.54 48.24) (width 0.2) (layer "F.Cu") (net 7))
 (segment (start 179.2 45.2) (end 178.125 46.275) (width 0.2) (layer "F.Cu") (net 7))
 (segment (start 151.54 48.24) (end 150.7 47.4) (width 0.2) (layer "F.Cu") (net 7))
 (via (at 166.6 36.9) (size 0.6) (drill 0.3) (layers "F.Cu" "B.Cu") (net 7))
 (via (at 179.2 45.2) (size 0.6) (drill 0.3) (layers "F.Cu" "B.Cu") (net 7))
 (segment (start 166.6 36.9) (end 172.2 36.9) (width 0.2) (layer "B.Cu") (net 7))
 (segment (start 179 45) (end 179.2 45.2) (width 0.2) (layer "B.Cu") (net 7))
 (segment (start 179 43.7) (end 179 45) (width 0.2) (layer "B.Cu") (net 7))
 (segment (start 172.2 36.9) (end 179 43.7) (width 0.2) (layer "B.Cu") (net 7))
 (segment (start 168.933626 53.32) (end 168.32 53.32) (width 0.2) (layer "F.Cu") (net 10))
 (segment (start 156.09 65.36) (end 161.65 59.8) (width 0.2) (layer "F.Cu") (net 10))
 (segment (start 161.65 59.8) (end 162.1 59.8) (width 0.2) (layer "F.Cu") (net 10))
 (via (at 162.1 59.8) (size 0.6) (drill 0.3) (layers "F.Cu" "B.Cu") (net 10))
 (via (at 168.5 54.2) (size 0.6) (drill 0.3) (layers "F.Cu" "B.Cu") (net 10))
 (segment (start 167.7 54.2) (end 168.5 54.2) (width 0.2) (layer "B.Cu") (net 10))
 (segment (start 162.1 59.8) (end 167.7 54.2) (width 0.2) (layer "B.Cu") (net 10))
 (segment (start 156.09 84.36) (end 158.74 84.36) (width 0.2) (layer "F.Cu") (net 11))
 (segment (start 156.09 84.36) (end 155.9 84.17) (width 0.2) (layer "F.Cu") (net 11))
 (segment (start 158.74 84.36) (end 158.8 84.3) (width 0.2) (layer "F.Cu") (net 11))
 (via (at 158.8 84.3) (size 0.6) (drill 0.3) (layers "F.Cu" "B.Cu") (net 11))
 (segment (start 169.383 51.843) (end 168.32 50.78) (width 0.2) (layer "B.Cu") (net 11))
 (segment (start 158.8 84.3) (end 158.8 83.478686) (width 0.2) (layer "B.Cu") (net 11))
 (segment (start 158.8 83.478686) (end 169.383 72.895686) (width 0.2) (layer "B.Cu") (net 11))
 (segment (start 169.383 72.895686) (end 169.383 51.843) (width 0.2) (layer "B.Cu") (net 11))
 (segment (start 175.19 78.09) (end 173 75.9) (width 0.2) (layer "F.Cu") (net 2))
 (segment (start 175.19 84.36) (end 175.19 78.09) (width 0.2) (layer "F.Cu") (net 2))
 (via (at 173 75.9) (size 0.6) (drill 0.3) (layers "F.Cu" "B.Cu") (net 2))
 (segment (start 173 75.9) (end 173 51.7) (width 0.2) (layer "B.Cu") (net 2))
 (segment (start 169.54 48.24) (end 168.32 48.24) (width 0.2) (layer "B.Cu") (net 2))
 (segment (start 173 51.7) (end 169.54 48.24) (width 0.2) (layer "B.Cu") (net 2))
 (segment (start 137.09 84.36) (end 137.09 70.31) (width 0.2) (layer "F.Cu") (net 12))
 (segment (start 150.4 57) (end 150.9 57.5) (width 0.2) (layer "F.Cu") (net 12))
 (segment (start 137.09 70.31) (end 150.4 57) (width 0.2) (layer "F.Cu") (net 12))
 (segment (start 150.9 57.5) (end 152.9 57.5) (width 0.2) (layer "F.Cu") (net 12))
 (via (at 152.9 57.5) (size 0.6) (drill 0.3) (layers "F.Cu" "B.Cu") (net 12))
 (segment (start 164.7 45.7) (end 168.32 45.7) (width 0.2) (layer "B.Cu") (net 12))
 (segment (start 152.9 57.5) (end 164.7 45.7) (width 0.2) (layer "B.Cu") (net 12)))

